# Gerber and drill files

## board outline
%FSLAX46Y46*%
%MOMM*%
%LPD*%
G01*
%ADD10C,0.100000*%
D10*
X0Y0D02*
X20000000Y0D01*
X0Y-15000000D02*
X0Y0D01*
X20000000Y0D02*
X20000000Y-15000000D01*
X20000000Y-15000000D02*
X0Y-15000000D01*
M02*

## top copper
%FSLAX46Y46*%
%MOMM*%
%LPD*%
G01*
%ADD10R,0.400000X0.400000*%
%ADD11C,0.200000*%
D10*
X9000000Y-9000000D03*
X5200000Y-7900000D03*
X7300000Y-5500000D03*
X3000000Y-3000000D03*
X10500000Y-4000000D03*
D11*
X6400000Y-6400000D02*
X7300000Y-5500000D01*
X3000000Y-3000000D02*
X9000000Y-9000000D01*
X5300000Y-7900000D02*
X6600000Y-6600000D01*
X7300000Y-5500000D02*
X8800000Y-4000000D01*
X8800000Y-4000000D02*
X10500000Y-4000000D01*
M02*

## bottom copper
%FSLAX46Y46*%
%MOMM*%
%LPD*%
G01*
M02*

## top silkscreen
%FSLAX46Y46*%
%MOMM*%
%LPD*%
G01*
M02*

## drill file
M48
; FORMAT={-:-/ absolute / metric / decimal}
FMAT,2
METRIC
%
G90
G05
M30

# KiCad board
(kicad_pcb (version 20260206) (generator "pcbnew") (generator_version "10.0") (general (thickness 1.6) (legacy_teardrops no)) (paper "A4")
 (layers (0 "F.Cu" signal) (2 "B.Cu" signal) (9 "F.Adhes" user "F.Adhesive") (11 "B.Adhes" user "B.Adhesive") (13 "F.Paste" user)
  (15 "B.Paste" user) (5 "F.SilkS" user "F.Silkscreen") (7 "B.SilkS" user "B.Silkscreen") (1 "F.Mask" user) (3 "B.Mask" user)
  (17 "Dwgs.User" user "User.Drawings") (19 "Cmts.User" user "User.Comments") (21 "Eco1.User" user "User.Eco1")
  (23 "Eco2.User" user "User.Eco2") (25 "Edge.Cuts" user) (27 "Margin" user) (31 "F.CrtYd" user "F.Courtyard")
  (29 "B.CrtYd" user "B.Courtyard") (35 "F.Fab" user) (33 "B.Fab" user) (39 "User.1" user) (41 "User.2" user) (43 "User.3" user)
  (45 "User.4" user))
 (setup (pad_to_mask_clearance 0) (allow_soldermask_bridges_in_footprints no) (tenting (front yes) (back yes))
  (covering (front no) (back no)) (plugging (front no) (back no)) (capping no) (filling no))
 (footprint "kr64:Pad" (layer "F.Cu") (at 9 9)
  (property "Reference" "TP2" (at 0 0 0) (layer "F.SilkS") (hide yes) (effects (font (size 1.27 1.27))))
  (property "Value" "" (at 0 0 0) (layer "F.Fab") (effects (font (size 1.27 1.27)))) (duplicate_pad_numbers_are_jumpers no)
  (pad "1" smd rect (at 0 0) (size 0.4 0.4) (layers "F.Cu" "F.Mask" "F.Paste") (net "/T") (thermal_bridge_angle 45)))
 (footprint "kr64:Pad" (layer "F.Cu") (at 5.2 7.9)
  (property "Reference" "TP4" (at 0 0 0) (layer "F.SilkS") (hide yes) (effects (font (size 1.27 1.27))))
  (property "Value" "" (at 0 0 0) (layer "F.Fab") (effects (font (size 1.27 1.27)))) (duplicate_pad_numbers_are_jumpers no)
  (pad "1" smd rect (at 0 0) (size 0.4 0.4) (layers "F.Cu" "F.Mask" "F.Paste") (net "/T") (thermal_bridge_angle 45)))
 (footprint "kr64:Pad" (layer "F.Cu") (at 7.3 5.5)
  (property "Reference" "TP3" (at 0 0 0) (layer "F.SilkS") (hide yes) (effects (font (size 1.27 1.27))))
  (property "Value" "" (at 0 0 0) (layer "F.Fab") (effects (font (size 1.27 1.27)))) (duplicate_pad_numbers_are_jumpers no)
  (pad "1" smd rect (at 0 0) (size 0.4 0.4) (layers "F.Cu" "F.Mask" "F.Paste") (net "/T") (thermal_bridge_angle 45)))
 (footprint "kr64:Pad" (layer "F.Cu") (at 3 3)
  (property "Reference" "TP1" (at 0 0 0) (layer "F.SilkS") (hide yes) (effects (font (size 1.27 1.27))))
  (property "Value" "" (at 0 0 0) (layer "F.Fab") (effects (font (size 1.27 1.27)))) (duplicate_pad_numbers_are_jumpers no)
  (pad "1" smd rect (at 0 0) (size 0.4 0.4) (layers "F.Cu" "F.Mask" "F.Paste") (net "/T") (thermal_bridge_angle 45)))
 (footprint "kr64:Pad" (layer "F.Cu") (at 10.5 4)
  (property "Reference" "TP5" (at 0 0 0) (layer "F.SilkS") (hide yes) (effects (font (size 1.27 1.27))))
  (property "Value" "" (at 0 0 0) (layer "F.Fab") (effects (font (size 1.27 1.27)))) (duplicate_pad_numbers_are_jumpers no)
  (pad "1" smd rect (at 0 0) (size 0.4 0.4) (layers "F.Cu" "F.Mask" "F.Paste") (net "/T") (thermal_bridge_angle 45)))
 (gr_line (start 0 0) (end 20 0) (stroke (width 0.1) (type default)) (layer "Edge.Cuts"))
 (gr_line (start 0 15) (end 0 0) (stroke (width 0.1) (type default)) (layer "Edge.Cuts"))
 (gr_line (start 20 0) (end 20 15) (stroke (width 0.1) (type default)) (layer "Edge.Cuts"))
 (gr_line (start 20 15) (end 0 15) (stroke (width 0.1) (type default)) (layer "Edge.Cuts"))
 (segment (start 6.4 6.4) (end 7.3 5.5) (width 0.2) (layer "F.Cu") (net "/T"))
 (segment (start 3 3) (end 9 9) (width 0.2) (layer "F.Cu") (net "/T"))
 (segment (start 5.3 7.9) (end 6.6 6.6) (width 0.2) (layer "F.Cu") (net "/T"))
 (segment (start 7.3 5.5) (end 8.8 4) (width 0.2) (layer "F.Cu") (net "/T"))
 (segment (start 8.8 4) (end 10.5 4) (width 0.2) (layer "F.Cu") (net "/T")))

